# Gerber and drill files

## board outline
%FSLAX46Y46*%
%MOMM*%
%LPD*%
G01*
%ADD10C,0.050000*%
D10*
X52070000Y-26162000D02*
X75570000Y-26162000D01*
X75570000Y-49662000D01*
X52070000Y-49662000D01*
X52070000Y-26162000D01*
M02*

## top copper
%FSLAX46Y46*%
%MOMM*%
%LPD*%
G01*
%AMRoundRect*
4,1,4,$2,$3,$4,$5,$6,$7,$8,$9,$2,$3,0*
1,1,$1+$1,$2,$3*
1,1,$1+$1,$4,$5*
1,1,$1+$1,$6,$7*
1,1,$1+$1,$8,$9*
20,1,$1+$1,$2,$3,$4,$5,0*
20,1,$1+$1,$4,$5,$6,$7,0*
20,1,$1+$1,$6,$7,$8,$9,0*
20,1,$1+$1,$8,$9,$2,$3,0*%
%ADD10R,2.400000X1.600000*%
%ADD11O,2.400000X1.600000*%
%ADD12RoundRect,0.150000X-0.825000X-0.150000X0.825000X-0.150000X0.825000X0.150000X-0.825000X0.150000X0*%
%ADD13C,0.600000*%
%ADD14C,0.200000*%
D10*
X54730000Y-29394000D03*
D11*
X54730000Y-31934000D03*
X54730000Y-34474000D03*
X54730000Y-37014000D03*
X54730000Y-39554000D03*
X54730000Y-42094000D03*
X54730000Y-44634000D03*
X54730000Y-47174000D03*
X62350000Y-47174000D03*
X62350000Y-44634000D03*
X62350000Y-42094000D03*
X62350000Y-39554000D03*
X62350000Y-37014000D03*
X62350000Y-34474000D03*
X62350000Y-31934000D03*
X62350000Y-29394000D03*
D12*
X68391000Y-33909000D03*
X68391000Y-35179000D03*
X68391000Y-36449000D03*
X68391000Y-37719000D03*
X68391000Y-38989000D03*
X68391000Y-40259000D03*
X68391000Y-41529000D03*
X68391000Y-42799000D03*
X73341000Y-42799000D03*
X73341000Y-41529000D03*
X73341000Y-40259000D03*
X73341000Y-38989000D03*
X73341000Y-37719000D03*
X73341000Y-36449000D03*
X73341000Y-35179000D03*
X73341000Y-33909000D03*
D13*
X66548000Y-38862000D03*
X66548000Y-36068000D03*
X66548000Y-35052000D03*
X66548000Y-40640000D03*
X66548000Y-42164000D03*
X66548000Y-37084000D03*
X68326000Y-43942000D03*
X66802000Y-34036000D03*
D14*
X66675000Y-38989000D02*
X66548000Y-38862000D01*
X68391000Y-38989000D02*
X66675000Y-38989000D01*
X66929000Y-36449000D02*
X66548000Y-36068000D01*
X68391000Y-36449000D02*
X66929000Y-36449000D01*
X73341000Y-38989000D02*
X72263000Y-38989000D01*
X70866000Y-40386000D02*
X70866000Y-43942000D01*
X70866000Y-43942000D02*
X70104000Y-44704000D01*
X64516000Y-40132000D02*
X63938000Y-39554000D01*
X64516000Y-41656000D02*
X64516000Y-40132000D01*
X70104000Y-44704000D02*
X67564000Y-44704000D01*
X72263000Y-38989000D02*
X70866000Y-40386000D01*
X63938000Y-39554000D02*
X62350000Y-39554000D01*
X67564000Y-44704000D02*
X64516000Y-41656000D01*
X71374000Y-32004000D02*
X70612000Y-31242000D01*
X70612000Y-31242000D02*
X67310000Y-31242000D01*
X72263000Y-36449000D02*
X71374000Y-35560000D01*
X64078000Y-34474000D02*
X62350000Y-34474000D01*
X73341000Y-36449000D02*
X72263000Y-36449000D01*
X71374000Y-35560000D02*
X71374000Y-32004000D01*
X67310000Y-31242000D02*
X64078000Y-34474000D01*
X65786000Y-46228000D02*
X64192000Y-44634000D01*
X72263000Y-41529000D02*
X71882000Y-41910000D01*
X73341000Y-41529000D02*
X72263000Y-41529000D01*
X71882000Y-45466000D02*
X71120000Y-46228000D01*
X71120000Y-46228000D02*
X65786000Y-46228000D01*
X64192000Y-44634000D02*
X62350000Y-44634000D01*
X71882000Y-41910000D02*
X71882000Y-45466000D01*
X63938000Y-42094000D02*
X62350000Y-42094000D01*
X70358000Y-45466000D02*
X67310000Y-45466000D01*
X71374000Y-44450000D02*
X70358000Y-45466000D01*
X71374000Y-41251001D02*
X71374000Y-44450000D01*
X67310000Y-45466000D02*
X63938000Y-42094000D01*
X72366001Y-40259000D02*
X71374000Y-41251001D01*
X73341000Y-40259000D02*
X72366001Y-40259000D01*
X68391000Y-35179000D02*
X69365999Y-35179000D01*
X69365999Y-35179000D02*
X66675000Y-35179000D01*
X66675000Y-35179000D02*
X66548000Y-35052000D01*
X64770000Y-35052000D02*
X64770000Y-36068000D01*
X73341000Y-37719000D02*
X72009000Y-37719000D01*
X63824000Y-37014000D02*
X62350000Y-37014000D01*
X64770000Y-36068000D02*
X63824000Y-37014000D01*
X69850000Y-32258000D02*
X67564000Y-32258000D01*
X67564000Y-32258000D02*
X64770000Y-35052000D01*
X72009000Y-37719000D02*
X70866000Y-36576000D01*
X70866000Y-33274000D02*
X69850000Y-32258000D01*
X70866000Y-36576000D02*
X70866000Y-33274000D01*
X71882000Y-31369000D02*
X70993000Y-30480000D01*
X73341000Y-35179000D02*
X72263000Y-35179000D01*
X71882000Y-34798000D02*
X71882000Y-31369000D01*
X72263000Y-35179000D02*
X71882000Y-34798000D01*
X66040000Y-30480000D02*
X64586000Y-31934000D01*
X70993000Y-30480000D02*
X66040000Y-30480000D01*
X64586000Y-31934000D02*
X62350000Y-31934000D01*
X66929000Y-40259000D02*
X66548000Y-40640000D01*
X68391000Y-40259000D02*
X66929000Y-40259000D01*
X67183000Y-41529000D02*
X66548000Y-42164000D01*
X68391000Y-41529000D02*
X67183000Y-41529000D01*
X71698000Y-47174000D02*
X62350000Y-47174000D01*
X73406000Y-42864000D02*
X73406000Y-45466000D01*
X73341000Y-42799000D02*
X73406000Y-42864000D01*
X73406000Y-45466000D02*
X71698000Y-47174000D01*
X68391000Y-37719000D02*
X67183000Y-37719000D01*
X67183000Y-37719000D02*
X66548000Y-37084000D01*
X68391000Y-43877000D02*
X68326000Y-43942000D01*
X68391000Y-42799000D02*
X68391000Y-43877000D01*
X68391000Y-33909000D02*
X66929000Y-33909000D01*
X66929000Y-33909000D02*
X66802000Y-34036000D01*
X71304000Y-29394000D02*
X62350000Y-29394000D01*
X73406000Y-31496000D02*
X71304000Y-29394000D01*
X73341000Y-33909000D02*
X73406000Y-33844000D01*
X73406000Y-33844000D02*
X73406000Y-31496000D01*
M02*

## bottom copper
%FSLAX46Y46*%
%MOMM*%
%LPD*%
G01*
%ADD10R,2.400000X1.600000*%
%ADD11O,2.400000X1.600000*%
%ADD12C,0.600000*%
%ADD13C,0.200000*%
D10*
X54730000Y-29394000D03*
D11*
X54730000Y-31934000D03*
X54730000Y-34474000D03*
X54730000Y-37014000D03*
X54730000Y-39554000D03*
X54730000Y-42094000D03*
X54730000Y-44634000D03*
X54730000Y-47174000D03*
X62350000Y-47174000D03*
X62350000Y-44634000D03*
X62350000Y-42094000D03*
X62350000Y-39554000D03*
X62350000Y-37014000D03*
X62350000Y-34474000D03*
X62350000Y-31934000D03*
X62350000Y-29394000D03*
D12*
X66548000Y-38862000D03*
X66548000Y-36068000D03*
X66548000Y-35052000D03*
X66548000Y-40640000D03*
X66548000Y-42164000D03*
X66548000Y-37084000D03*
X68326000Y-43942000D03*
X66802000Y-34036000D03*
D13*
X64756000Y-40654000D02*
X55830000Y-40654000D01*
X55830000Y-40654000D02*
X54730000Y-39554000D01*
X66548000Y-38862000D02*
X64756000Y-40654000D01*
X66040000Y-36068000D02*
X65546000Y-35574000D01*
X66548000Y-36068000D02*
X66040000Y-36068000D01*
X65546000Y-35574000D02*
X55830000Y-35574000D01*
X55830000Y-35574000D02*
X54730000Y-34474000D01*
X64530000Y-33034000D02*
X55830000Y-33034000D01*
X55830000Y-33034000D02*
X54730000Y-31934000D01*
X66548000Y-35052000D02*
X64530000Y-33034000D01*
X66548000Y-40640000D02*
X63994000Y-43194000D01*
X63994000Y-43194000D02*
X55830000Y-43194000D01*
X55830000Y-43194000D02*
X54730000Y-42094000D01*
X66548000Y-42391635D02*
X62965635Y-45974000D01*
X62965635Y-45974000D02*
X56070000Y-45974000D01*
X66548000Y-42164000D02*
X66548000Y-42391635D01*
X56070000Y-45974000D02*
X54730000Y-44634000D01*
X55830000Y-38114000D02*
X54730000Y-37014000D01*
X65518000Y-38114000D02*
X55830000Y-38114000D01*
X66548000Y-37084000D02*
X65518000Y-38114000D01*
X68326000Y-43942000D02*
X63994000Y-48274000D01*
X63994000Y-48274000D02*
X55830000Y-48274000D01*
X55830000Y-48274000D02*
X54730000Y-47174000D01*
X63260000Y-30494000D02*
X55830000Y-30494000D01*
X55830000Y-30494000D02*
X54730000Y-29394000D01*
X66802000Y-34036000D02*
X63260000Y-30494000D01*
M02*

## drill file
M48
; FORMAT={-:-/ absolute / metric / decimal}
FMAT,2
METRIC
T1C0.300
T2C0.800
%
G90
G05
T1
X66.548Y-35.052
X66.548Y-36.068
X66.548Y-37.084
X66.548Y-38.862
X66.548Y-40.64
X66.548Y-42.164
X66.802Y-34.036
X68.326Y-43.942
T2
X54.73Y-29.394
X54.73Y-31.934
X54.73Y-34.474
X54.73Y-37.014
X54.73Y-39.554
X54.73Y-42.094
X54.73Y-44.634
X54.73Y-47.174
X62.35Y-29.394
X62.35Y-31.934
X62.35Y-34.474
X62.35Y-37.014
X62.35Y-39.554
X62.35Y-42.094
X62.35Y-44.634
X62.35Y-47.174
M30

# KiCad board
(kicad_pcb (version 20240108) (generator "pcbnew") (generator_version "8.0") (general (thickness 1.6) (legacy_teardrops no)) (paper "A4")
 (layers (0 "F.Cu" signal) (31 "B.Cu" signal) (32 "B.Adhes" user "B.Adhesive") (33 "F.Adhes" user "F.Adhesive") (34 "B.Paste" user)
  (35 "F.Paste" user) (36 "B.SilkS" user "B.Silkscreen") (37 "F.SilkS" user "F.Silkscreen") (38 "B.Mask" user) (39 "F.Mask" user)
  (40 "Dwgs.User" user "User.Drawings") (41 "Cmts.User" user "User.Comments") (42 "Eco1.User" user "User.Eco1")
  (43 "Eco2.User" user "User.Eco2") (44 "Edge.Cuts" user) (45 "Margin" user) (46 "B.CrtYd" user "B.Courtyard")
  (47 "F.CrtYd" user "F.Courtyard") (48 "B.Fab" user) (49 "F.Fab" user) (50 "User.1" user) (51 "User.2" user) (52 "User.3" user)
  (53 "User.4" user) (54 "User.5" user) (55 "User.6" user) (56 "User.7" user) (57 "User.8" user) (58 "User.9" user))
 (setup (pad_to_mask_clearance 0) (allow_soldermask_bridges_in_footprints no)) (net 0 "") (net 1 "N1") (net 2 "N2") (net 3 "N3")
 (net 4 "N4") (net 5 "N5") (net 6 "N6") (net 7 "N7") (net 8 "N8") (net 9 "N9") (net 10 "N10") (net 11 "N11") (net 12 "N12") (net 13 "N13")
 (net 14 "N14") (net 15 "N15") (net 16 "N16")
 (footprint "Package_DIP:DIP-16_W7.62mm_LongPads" (layer "F.Cu") (at 54.73 29.394)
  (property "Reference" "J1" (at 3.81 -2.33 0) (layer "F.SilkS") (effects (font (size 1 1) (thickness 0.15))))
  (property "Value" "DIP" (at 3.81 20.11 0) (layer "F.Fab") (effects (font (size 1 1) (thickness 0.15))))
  (pad "1" thru_hole rect (at 0 0) (size 2.4 1.6) (drill 0.8) (layers "*.Cu" "*.Mask") (remove_unused_layers no) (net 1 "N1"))
  (pad "2" thru_hole oval (at 0 2.54) (size 2.4 1.6) (drill 0.8) (layers "*.Cu" "*.Mask") (remove_unused_layers no) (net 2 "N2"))
  (pad "3" thru_hole oval (at 0 5.08) (size 2.4 1.6) (drill 0.8) (layers "*.Cu" "*.Mask") (remove_unused_layers no) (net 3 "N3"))
  (pad "4" thru_hole oval (at 0 7.62) (size 2.4 1.6) (drill 0.8) (layers "*.Cu" "*.Mask") (remove_unused_layers no) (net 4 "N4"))
  (pad "5" thru_hole oval (at 0 10.16) (size 2.4 1.6) (drill 0.8) (layers "*.Cu" "*.Mask") (remove_unused_layers no) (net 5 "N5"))
  (pad "6" thru_hole oval (at 0 12.7) (size 2.4 1.6) (drill 0.8) (layers "*.Cu" "*.Mask") (remove_unused_layers no) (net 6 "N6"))
  (pad "7" thru_hole oval (at 0 15.24) (size 2.4 1.6) (drill 0.8) (layers "*.Cu" "*.Mask") (remove_unused_layers no) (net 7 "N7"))
  (pad "8" thru_hole oval (at 0 17.78) (size 2.4 1.6) (drill 0.8) (layers "*.Cu" "*.Mask") (remove_unused_layers no) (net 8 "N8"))
  (pad "9" thru_hole oval (at 7.62 17.78) (size 2.4 1.6) (drill 0.8) (layers "*.Cu" "*.Mask") (remove_unused_layers no) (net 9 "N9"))
  (pad "10" thru_hole oval (at 7.62 15.24) (size 2.4 1.6) (drill 0.8) (layers "*.Cu" "*.Mask") (remove_unused_layers no) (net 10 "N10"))
  (pad "11" thru_hole oval (at 7.62 12.7) (size 2.4 1.6) (drill 0.8) (layers "*.Cu" "*.Mask") (remove_unused_layers no) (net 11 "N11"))
  (pad "12" thru_hole oval (at 7.62 10.16) (size 2.4 1.6) (drill 0.8) (layers "*.Cu" "*.Mask") (remove_unused_layers no) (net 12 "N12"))
  (pad "13" thru_hole oval (at 7.62 7.62) (size 2.4 1.6) (drill 0.8) (layers "*.Cu" "*.Mask") (remove_unused_layers no) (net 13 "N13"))
  (pad "14" thru_hole oval (at 7.62 5.08) (size 2.4 1.6) (drill 0.8) (layers "*.Cu" "*.Mask") (remove_unused_layers no) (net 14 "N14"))
  (pad "15" thru_hole oval (at 7.62 2.54) (size 2.4 1.6) (drill 0.8) (layers "*.Cu" "*.Mask") (remove_unused_layers no) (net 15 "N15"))
  (pad "16" thru_hole oval (at 7.62 0) (size 2.4 1.6) (drill 0.8) (layers "*.Cu" "*.Mask") (remove_unused_layers no) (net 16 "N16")))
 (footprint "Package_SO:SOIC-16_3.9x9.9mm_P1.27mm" (layer "F.Cu") (at 70.866 38.354)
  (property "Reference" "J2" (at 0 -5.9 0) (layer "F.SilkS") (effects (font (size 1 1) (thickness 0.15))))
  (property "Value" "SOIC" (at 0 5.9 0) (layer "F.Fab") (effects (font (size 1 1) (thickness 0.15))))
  (pad "1" smd roundrect (at -2.475 -4.445) (size 1.95 0.6) (layers "F.Cu" "F.Paste" "F.Mask") (roundrect_rratio 0.25) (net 1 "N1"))
  (pad "2" smd roundrect (at -2.475 -3.175) (size 1.95 0.6) (layers "F.Cu" "F.Paste" "F.Mask") (roundrect_rratio 0.25) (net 2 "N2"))
  (pad "3" smd roundrect (at -2.475 -1.905) (size 1.95 0.6) (layers "F.Cu" "F.Paste" "F.Mask") (roundrect_rratio 0.25) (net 3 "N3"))
  (pad "4" smd roundrect (at -2.475 -0.635) (size 1.95 0.6) (layers "F.Cu" "F.Paste" "F.Mask") (roundrect_rratio 0.25) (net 4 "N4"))
  (pad "5" smd roundrect (at -2.475 0.635) (size 1.95 0.6) (layers "F.Cu" "F.Paste" "F.Mask") (roundrect_rratio 0.25) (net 5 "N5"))
  (pad "6" smd roundrect (at -2.475 1.905) (size 1.95 0.6) (layers "F.Cu" "F.Paste" "F.Mask") (roundrect_rratio 0.25) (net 6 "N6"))
  (pad "7" smd roundrect (at -2.475 3.175) (size 1.95 0.6) (layers "F.Cu" "F.Paste" "F.Mask") (roundrect_rratio 0.25) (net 7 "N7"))
  (pad "8" smd roundrect (at -2.475 4.445) (size 1.95 0.6) (layers "F.Cu" "F.Paste" "F.Mask") (roundrect_rratio 0.25) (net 8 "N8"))
  (pad "9" smd roundrect (at 2.475 4.445) (size 1.95 0.6) (layers "F.Cu" "F.Paste" "F.Mask") (roundrect_rratio 0.25) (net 9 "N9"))
  (pad "10" smd roundrect (at 2.475 3.175) (size 1.95 0.6) (layers "F.Cu" "F.Paste" "F.Mask") (roundrect_rratio 0.25) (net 10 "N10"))
  (pad "11" smd roundrect (at 2.475 1.905) (size 1.95 0.6) (layers "F.Cu" "F.Paste" "F.Mask") (roundrect_rratio 0.25) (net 11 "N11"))
  (pad "12" smd roundrect (at 2.475 0.635) (size 1.95 0.6) (layers "F.Cu" "F.Paste" "F.Mask") (roundrect_rratio 0.25) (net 12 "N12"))
  (pad "13" smd roundrect (at 2.475 -0.635) (size 1.95 0.6) (layers "F.Cu" "F.Paste" "F.Mask") (roundrect_rratio 0.25) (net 13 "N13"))
  (pad "14" smd roundrect (at 2.475 -1.905) (size 1.95 0.6) (layers "F.Cu" "F.Paste" "F.Mask") (roundrect_rratio 0.25) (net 14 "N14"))
  (pad "15" smd roundrect (at 2.475 -3.175) (size 1.95 0.6) (layers "F.Cu" "F.Paste" "F.Mask") (roundrect_rratio 0.25) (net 15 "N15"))
  (pad "16" smd roundrect (at 2.475 -4.445) (size 1.95 0.6) (layers "F.Cu" "F.Paste" "F.Mask") (roundrect_rratio 0.25) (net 16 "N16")))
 (gr_rect (start 52.07 26.162) (end 75.57 49.662) (stroke (width 0.05) (type default)) (fill none) (layer "Edge.Cuts"))
 (segment (start 66.675 38.989) (end 66.548 38.862) (width 0.2) (layer "F.Cu") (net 5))
 (segment (start 68.391 38.989) (end 66.675 38.989) (width 0.2) (layer "F.Cu") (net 5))
 (via (at 66.548 38.862) (size 0.6) (drill 0.3) (layers "F.Cu" "B.Cu") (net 5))
 (segment (start 64.756 40.654) (end 55.83 40.654) (width 0.2) (layer "B.Cu") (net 5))
 (segment (start 55.83 40.654) (end 54.73 39.554) (width 0.2) (layer "B.Cu") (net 5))
 (segment (start 66.548 38.862) (end 64.756 40.654) (width 0.2) (layer "B.Cu") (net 5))
 (segment (start 66.929 36.449) (end 66.548 36.068) (width 0.2) (layer "F.Cu") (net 3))
 (segment (start 68.391 36.449) (end 66.929 36.449) (width 0.2) (layer "F.Cu") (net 3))
 (via (at 66.548 36.068) (size 0.6) (drill 0.3) (layers "F.Cu" "B.Cu") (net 3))
 (segment (start 66.04 36.068) (end 65.546 35.574) (width 0.2) (layer "B.Cu") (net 3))
 (segment (start 66.548 36.068) (end 66.04 36.068) (width 0.2) (layer "B.Cu") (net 3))
 (segment (start 65.546 35.574) (end 55.83 35.574) (width 0.2) (layer "B.Cu") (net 3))
 (segment (start 55.83 35.574) (end 54.73 34.474) (width 0.2) (layer "B.Cu") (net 3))
 (segment (start 73.341 38.989) (end 72.263 38.989) (width 0.2) (layer "F.Cu") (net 12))
 (segment (start 70.866 40.386) (end 70.866 43.942) (width 0.2) (layer "F.Cu") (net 12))
 (segment (start 70.866 43.942) (end 70.104 44.704) (width 0.2) (layer "F.Cu") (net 12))
 (segment (start 64.516 40.132) (end 63.938 39.554) (width 0.2) (layer "F.Cu") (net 12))
 (segment (start 64.516 41.656) (end 64.516 40.132) (width 0.2) (layer "F.Cu") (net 12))
 (segment (start 70.104 44.704) (end 67.564 44.704) (width 0.2) (layer "F.Cu") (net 12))
 (segment (start 72.263 38.989) (end 70.866 40.386) (width 0.2) (layer "F.Cu") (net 12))
 (segment (start 63.938 39.554) (end 62.35 39.554) (width 0.2) (layer "F.Cu") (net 12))
 (segment (start 67.564 44.704) (end 64.516 41.656) (width 0.2) (layer "F.Cu") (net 12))
 (segment (start 71.374 32.004) (end 70.612 31.242) (width 0.2) (layer "F.Cu") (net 14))
 (segment (start 70.612 31.242) (end 67.31 31.242) (width 0.2) (layer "F.Cu") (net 14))
 (segment (start 72.263 36.449) (end 71.374 35.56) (width 0.2) (layer "F.Cu") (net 14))
 (segment (start 64.078 34.474) (end 62.35 34.474) (width 0.2) (layer "F.Cu") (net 14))
 (segment (start 73.341 36.449) (end 72.263 36.449) (width 0.2) (layer "F.Cu") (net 14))
 (segment (start 71.374 35.56) (end 71.374 32.004) (width 0.2) (layer "F.Cu") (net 14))
 (segment (start 67.31 31.242) (end 64.078 34.474) (width 0.2) (layer "F.Cu") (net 14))
 (segment (start 65.786 46.228) (end 64.192 44.634) (width 0.2) (layer "F.Cu") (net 10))
 (segment (start 72.263 41.529) (end 71.882 41.91) (width 0.2) (layer "F.Cu") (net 10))
 (segment (start 73.341 41.529) (end 72.263 41.529) (width 0.2) (layer "F.Cu") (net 10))
 (segment (start 71.882 45.466) (end 71.12 46.228) (width 0.2) (layer "F.Cu") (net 10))
 (segment (start 71.12 46.228) (end 65.786 46.228) (width 0.2) (layer "F.Cu") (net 10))
 (segment (start 64.192 44.634) (end 62.35 44.634) (width 0.2) (layer "F.Cu") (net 10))
 (segment (start 71.882 41.91) (end 71.882 45.466) (width 0.2) (layer "F.Cu") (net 10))
 (segment (start 63.938 42.094) (end 62.35 42.094) (width 0.2) (layer "F.Cu") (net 11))
 (segment (start 70.358 45.466) (end 67.31 45.466) (width 0.2) (layer "F.Cu") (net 11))
 (segment (start 71.374 44.45) (end 70.358 45.466) (width 0.2) (layer "F.Cu") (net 11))
 (segment (start 71.374 41.251001) (end 71.374 44.45) (width 0.2) (layer "F.Cu") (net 11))
 (segment (start 67.31 45.466) (end 63.938 42.094) (width 0.2) (layer "F.Cu") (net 11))
 (segment (start 72.366001 40.259) (end 71.374 41.251001) (width 0.2) (layer "F.Cu") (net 11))
 (segment (start 73.341 40.259) (end 72.366001 40.259) (width 0.2) (layer "F.Cu") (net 11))
 (segment (start 68.391 35.179) (end 69.365999 35.179) (width 0.2) (layer "F.Cu") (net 2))
 (segment (start 69.365999 35.179) (end 66.675 35.179) (width 0.2) (layer "F.Cu") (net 2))
 (segment (start 66.675 35.179) (end 66.548 35.052) (width 0.2) (layer "F.Cu") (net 2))
 (via (at 66.548 35.052) (size 0.6) (drill 0.3) (layers "F.Cu" "B.Cu") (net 2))
 (segment (start 64.53 33.034) (end 55.83 33.034) (width 0.2) (layer "B.Cu") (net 2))
 (segment (start 55.83 33.034) (end 54.73 31.934) (width 0.2) (layer "B.Cu") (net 2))
 (segment (start 66.548 35.052) (end 64.53 33.034) (width 0.2) (layer "B.Cu") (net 2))
 (segment (start 64.77 35.052) (end 64.77 36.068) (width 0.2) (layer "F.Cu") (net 13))
 (segment (start 73.341 37.719) (end 72.009 37.719) (width 0.2) (layer "F.Cu") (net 13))
 (segment (start 63.824 37.014) (end 62.35 37.014) (width 0.2) (layer "F.Cu") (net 13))
 (segment (start 64.77 36.068) (end 63.824 37.014) (width 0.2) (layer "F.Cu") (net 13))
 (segment (start 69.85 32.258) (end 67.564 32.258) (width 0.2) (layer "F.Cu") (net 13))
 (segment (start 67.564 32.258) (end 64.77 35.052) (width 0.2) (layer "F.Cu") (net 13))
 (segment (start 72.009 37.719) (end 70.866 36.576) (width 0.2) (layer "F.Cu") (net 13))
 (segment (start 70.866 33.274) (end 69.85 32.258) (width 0.2) (layer "F.Cu") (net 13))
 (segment (start 70.866 36.576) (end 70.866 33.274) (width 0.2) (layer "F.Cu") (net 13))
 (segment (start 71.882 31.369) (end 70.993 30.48) (width 0.2) (layer "F.Cu") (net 15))
 (segment (start 73.341 35.179) (end 72.263 35.179) (width 0.2) (layer "F.Cu") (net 15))
 (segment (start 71.882 34.798) (end 71.882 31.369) (width 0.2) (layer "F.Cu") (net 15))
 (segment (start 72.263 35.179) (end 71.882 34.798) (width 0.2) (layer "F.Cu") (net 15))
 (segment (start 66.04 30.48) (end 64.586 31.934) (width 0.2) (layer "F.Cu") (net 15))
 (segment (start 70.993 30.48) (end 66.04 30.48) (width 0.2) (layer "F.Cu") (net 15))
 (segment (start 64.586 31.934) (end 62.35 31.934) (width 0.2) (layer "F.Cu") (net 15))
 (segment (start 66.929 40.259) (end 66.548 40.64) (width 0.2) (layer "F.Cu") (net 6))
 (segment (start 68.391 40.259) (end 66.929 40.259) (width 0.2) (layer "F.Cu") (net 6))
 (via (at 66.548 40.64) (size 0.6) (drill 0.3) (layers "F.Cu" "B.Cu") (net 6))
 (segment (start 66.548 40.64) (end 63.994 43.194) (width 0.2) (layer "B.Cu") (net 6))
 (segment (start 63.994 43.194) (end 55.83 43.194) (width 0.2) (layer "B.Cu") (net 6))
 (segment (start 55.83 43.194) (end 54.73 42.094) (width 0.2) (layer "B.Cu") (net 6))
 (segment (start 67.183 41.529) (end 66.548 42.164) (width 0.2) (layer "F.Cu") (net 7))
 (segment (start 68.391 41.529) (end 67.183 41.529) (width 0.2) (layer "F.Cu") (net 7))
 (via (at 66.548 42.164) (size 0.6) (drill 0.3) (layers "F.Cu" "B.Cu") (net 7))
 (segment (start 66.548 42.391635) (end 62.965635 45.974) (width 0.2) (layer "B.Cu") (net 7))
 (segment (start 62.965635 45.974) (end 56.07 45.974) (width 0.2) (layer "B.Cu") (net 7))
 (segment (start 66.548 42.164) (end 66.548 42.391635) (width 0.2) (layer "B.Cu") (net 7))
 (segment (start 56.07 45.974) (end 54.73 44.634) (width 0.2) (layer "B.Cu") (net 7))
 (segment (start 71.698 47.174) (end 62.35 47.174) (width 0.2) (layer "F.Cu") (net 9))
 (segment (start 73.406 42.864) (end 73.406 45.466) (width 0.2) (layer "F.Cu") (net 9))
 (segment (start 73.341 42.799) (end 73.406 42.864) (width 0.2) (layer "F.Cu") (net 9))
 (segment (start 73.406 45.466) (end 71.698 47.174) (width 0.2) (layer "F.Cu") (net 9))
 (segment (start 68.391 37.719) (end 67.183 37.719) (width 0.2) (layer "F.Cu") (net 4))
 (segment (start 67.183 37.719) (end 66.548 37.084) (width 0.2) (layer "F.Cu") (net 4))
 (via (at 66.548 37.084) (size 0.6) (drill 0.3) (layers "F.Cu" "B.Cu") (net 4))
 (segment (start 55.83 38.114) (end 54.73 37.014) (width 0.2) (layer "B.Cu") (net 4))
 (segment (start 65.518 38.114) (end 55.83 38.114) (width 0.2) (layer "B.Cu") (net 4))
 (segment (start 66.548 37.084) (end 65.518 38.114) (width 0.2) (layer "B.Cu") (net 4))
 (segment (start 68.391 43.877) (end 68.326 43.942) (width 0.2) (layer "F.Cu") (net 8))
 (segment (start 68.391 42.799) (end 68.391 43.877) (width 0.2) (layer "F.Cu") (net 8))
 (via (at 68.326 43.942) (size 0.6) (drill 0.3) (layers "F.Cu" "B.Cu") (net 8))
 (segment (start 68.326 43.942) (end 63.994 48.274) (width 0.2) (layer "B.Cu") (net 8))
 (segment (start 63.994 48.274) (end 55.83 48.274) (width 0.2) (layer "B.Cu") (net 8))
 (segment (start 55.83 48.274) (end 54.73 47.174) (width 0.2) (layer "B.Cu") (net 8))
 (segment (start 68.391 33.909) (end 66.929 33.909) (width 0.2) (layer "F.Cu") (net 1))
 (segment (start 66.929 33.909) (end 66.802 34.036) (width 0.2) (layer "F.Cu") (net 1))
 (via (at 66.802 34.036) (size 0.6) (drill 0.3) (layers "F.Cu" "B.Cu") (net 1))
 (segment (start 63.26 30.494) (end 55.83 30.494) (width 0.2) (layer "B.Cu") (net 1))
 (segment (start 55.83 30.494) (end 54.73 29.394) (width 0.2) (layer "B.Cu") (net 1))
 (segment (start 66.802 34.036) (end 63.26 30.494) (width 0.2) (layer "B.Cu") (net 1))
 (segment (start 71.304 29.394) (end 62.35 29.394) (width 0.2) (layer "F.Cu") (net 16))
 (segment (start 73.406 31.496) (end 71.304 29.394) (width 0.2) (layer "F.Cu") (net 16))
 (segment (start 73.341 33.909) (end 73.406 33.844) (width 0.2) (layer "F.Cu") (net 16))
 (segment (start 73.406 33.844) (end 73.406 31.496) (width 0.2) (layer "F.Cu") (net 16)))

